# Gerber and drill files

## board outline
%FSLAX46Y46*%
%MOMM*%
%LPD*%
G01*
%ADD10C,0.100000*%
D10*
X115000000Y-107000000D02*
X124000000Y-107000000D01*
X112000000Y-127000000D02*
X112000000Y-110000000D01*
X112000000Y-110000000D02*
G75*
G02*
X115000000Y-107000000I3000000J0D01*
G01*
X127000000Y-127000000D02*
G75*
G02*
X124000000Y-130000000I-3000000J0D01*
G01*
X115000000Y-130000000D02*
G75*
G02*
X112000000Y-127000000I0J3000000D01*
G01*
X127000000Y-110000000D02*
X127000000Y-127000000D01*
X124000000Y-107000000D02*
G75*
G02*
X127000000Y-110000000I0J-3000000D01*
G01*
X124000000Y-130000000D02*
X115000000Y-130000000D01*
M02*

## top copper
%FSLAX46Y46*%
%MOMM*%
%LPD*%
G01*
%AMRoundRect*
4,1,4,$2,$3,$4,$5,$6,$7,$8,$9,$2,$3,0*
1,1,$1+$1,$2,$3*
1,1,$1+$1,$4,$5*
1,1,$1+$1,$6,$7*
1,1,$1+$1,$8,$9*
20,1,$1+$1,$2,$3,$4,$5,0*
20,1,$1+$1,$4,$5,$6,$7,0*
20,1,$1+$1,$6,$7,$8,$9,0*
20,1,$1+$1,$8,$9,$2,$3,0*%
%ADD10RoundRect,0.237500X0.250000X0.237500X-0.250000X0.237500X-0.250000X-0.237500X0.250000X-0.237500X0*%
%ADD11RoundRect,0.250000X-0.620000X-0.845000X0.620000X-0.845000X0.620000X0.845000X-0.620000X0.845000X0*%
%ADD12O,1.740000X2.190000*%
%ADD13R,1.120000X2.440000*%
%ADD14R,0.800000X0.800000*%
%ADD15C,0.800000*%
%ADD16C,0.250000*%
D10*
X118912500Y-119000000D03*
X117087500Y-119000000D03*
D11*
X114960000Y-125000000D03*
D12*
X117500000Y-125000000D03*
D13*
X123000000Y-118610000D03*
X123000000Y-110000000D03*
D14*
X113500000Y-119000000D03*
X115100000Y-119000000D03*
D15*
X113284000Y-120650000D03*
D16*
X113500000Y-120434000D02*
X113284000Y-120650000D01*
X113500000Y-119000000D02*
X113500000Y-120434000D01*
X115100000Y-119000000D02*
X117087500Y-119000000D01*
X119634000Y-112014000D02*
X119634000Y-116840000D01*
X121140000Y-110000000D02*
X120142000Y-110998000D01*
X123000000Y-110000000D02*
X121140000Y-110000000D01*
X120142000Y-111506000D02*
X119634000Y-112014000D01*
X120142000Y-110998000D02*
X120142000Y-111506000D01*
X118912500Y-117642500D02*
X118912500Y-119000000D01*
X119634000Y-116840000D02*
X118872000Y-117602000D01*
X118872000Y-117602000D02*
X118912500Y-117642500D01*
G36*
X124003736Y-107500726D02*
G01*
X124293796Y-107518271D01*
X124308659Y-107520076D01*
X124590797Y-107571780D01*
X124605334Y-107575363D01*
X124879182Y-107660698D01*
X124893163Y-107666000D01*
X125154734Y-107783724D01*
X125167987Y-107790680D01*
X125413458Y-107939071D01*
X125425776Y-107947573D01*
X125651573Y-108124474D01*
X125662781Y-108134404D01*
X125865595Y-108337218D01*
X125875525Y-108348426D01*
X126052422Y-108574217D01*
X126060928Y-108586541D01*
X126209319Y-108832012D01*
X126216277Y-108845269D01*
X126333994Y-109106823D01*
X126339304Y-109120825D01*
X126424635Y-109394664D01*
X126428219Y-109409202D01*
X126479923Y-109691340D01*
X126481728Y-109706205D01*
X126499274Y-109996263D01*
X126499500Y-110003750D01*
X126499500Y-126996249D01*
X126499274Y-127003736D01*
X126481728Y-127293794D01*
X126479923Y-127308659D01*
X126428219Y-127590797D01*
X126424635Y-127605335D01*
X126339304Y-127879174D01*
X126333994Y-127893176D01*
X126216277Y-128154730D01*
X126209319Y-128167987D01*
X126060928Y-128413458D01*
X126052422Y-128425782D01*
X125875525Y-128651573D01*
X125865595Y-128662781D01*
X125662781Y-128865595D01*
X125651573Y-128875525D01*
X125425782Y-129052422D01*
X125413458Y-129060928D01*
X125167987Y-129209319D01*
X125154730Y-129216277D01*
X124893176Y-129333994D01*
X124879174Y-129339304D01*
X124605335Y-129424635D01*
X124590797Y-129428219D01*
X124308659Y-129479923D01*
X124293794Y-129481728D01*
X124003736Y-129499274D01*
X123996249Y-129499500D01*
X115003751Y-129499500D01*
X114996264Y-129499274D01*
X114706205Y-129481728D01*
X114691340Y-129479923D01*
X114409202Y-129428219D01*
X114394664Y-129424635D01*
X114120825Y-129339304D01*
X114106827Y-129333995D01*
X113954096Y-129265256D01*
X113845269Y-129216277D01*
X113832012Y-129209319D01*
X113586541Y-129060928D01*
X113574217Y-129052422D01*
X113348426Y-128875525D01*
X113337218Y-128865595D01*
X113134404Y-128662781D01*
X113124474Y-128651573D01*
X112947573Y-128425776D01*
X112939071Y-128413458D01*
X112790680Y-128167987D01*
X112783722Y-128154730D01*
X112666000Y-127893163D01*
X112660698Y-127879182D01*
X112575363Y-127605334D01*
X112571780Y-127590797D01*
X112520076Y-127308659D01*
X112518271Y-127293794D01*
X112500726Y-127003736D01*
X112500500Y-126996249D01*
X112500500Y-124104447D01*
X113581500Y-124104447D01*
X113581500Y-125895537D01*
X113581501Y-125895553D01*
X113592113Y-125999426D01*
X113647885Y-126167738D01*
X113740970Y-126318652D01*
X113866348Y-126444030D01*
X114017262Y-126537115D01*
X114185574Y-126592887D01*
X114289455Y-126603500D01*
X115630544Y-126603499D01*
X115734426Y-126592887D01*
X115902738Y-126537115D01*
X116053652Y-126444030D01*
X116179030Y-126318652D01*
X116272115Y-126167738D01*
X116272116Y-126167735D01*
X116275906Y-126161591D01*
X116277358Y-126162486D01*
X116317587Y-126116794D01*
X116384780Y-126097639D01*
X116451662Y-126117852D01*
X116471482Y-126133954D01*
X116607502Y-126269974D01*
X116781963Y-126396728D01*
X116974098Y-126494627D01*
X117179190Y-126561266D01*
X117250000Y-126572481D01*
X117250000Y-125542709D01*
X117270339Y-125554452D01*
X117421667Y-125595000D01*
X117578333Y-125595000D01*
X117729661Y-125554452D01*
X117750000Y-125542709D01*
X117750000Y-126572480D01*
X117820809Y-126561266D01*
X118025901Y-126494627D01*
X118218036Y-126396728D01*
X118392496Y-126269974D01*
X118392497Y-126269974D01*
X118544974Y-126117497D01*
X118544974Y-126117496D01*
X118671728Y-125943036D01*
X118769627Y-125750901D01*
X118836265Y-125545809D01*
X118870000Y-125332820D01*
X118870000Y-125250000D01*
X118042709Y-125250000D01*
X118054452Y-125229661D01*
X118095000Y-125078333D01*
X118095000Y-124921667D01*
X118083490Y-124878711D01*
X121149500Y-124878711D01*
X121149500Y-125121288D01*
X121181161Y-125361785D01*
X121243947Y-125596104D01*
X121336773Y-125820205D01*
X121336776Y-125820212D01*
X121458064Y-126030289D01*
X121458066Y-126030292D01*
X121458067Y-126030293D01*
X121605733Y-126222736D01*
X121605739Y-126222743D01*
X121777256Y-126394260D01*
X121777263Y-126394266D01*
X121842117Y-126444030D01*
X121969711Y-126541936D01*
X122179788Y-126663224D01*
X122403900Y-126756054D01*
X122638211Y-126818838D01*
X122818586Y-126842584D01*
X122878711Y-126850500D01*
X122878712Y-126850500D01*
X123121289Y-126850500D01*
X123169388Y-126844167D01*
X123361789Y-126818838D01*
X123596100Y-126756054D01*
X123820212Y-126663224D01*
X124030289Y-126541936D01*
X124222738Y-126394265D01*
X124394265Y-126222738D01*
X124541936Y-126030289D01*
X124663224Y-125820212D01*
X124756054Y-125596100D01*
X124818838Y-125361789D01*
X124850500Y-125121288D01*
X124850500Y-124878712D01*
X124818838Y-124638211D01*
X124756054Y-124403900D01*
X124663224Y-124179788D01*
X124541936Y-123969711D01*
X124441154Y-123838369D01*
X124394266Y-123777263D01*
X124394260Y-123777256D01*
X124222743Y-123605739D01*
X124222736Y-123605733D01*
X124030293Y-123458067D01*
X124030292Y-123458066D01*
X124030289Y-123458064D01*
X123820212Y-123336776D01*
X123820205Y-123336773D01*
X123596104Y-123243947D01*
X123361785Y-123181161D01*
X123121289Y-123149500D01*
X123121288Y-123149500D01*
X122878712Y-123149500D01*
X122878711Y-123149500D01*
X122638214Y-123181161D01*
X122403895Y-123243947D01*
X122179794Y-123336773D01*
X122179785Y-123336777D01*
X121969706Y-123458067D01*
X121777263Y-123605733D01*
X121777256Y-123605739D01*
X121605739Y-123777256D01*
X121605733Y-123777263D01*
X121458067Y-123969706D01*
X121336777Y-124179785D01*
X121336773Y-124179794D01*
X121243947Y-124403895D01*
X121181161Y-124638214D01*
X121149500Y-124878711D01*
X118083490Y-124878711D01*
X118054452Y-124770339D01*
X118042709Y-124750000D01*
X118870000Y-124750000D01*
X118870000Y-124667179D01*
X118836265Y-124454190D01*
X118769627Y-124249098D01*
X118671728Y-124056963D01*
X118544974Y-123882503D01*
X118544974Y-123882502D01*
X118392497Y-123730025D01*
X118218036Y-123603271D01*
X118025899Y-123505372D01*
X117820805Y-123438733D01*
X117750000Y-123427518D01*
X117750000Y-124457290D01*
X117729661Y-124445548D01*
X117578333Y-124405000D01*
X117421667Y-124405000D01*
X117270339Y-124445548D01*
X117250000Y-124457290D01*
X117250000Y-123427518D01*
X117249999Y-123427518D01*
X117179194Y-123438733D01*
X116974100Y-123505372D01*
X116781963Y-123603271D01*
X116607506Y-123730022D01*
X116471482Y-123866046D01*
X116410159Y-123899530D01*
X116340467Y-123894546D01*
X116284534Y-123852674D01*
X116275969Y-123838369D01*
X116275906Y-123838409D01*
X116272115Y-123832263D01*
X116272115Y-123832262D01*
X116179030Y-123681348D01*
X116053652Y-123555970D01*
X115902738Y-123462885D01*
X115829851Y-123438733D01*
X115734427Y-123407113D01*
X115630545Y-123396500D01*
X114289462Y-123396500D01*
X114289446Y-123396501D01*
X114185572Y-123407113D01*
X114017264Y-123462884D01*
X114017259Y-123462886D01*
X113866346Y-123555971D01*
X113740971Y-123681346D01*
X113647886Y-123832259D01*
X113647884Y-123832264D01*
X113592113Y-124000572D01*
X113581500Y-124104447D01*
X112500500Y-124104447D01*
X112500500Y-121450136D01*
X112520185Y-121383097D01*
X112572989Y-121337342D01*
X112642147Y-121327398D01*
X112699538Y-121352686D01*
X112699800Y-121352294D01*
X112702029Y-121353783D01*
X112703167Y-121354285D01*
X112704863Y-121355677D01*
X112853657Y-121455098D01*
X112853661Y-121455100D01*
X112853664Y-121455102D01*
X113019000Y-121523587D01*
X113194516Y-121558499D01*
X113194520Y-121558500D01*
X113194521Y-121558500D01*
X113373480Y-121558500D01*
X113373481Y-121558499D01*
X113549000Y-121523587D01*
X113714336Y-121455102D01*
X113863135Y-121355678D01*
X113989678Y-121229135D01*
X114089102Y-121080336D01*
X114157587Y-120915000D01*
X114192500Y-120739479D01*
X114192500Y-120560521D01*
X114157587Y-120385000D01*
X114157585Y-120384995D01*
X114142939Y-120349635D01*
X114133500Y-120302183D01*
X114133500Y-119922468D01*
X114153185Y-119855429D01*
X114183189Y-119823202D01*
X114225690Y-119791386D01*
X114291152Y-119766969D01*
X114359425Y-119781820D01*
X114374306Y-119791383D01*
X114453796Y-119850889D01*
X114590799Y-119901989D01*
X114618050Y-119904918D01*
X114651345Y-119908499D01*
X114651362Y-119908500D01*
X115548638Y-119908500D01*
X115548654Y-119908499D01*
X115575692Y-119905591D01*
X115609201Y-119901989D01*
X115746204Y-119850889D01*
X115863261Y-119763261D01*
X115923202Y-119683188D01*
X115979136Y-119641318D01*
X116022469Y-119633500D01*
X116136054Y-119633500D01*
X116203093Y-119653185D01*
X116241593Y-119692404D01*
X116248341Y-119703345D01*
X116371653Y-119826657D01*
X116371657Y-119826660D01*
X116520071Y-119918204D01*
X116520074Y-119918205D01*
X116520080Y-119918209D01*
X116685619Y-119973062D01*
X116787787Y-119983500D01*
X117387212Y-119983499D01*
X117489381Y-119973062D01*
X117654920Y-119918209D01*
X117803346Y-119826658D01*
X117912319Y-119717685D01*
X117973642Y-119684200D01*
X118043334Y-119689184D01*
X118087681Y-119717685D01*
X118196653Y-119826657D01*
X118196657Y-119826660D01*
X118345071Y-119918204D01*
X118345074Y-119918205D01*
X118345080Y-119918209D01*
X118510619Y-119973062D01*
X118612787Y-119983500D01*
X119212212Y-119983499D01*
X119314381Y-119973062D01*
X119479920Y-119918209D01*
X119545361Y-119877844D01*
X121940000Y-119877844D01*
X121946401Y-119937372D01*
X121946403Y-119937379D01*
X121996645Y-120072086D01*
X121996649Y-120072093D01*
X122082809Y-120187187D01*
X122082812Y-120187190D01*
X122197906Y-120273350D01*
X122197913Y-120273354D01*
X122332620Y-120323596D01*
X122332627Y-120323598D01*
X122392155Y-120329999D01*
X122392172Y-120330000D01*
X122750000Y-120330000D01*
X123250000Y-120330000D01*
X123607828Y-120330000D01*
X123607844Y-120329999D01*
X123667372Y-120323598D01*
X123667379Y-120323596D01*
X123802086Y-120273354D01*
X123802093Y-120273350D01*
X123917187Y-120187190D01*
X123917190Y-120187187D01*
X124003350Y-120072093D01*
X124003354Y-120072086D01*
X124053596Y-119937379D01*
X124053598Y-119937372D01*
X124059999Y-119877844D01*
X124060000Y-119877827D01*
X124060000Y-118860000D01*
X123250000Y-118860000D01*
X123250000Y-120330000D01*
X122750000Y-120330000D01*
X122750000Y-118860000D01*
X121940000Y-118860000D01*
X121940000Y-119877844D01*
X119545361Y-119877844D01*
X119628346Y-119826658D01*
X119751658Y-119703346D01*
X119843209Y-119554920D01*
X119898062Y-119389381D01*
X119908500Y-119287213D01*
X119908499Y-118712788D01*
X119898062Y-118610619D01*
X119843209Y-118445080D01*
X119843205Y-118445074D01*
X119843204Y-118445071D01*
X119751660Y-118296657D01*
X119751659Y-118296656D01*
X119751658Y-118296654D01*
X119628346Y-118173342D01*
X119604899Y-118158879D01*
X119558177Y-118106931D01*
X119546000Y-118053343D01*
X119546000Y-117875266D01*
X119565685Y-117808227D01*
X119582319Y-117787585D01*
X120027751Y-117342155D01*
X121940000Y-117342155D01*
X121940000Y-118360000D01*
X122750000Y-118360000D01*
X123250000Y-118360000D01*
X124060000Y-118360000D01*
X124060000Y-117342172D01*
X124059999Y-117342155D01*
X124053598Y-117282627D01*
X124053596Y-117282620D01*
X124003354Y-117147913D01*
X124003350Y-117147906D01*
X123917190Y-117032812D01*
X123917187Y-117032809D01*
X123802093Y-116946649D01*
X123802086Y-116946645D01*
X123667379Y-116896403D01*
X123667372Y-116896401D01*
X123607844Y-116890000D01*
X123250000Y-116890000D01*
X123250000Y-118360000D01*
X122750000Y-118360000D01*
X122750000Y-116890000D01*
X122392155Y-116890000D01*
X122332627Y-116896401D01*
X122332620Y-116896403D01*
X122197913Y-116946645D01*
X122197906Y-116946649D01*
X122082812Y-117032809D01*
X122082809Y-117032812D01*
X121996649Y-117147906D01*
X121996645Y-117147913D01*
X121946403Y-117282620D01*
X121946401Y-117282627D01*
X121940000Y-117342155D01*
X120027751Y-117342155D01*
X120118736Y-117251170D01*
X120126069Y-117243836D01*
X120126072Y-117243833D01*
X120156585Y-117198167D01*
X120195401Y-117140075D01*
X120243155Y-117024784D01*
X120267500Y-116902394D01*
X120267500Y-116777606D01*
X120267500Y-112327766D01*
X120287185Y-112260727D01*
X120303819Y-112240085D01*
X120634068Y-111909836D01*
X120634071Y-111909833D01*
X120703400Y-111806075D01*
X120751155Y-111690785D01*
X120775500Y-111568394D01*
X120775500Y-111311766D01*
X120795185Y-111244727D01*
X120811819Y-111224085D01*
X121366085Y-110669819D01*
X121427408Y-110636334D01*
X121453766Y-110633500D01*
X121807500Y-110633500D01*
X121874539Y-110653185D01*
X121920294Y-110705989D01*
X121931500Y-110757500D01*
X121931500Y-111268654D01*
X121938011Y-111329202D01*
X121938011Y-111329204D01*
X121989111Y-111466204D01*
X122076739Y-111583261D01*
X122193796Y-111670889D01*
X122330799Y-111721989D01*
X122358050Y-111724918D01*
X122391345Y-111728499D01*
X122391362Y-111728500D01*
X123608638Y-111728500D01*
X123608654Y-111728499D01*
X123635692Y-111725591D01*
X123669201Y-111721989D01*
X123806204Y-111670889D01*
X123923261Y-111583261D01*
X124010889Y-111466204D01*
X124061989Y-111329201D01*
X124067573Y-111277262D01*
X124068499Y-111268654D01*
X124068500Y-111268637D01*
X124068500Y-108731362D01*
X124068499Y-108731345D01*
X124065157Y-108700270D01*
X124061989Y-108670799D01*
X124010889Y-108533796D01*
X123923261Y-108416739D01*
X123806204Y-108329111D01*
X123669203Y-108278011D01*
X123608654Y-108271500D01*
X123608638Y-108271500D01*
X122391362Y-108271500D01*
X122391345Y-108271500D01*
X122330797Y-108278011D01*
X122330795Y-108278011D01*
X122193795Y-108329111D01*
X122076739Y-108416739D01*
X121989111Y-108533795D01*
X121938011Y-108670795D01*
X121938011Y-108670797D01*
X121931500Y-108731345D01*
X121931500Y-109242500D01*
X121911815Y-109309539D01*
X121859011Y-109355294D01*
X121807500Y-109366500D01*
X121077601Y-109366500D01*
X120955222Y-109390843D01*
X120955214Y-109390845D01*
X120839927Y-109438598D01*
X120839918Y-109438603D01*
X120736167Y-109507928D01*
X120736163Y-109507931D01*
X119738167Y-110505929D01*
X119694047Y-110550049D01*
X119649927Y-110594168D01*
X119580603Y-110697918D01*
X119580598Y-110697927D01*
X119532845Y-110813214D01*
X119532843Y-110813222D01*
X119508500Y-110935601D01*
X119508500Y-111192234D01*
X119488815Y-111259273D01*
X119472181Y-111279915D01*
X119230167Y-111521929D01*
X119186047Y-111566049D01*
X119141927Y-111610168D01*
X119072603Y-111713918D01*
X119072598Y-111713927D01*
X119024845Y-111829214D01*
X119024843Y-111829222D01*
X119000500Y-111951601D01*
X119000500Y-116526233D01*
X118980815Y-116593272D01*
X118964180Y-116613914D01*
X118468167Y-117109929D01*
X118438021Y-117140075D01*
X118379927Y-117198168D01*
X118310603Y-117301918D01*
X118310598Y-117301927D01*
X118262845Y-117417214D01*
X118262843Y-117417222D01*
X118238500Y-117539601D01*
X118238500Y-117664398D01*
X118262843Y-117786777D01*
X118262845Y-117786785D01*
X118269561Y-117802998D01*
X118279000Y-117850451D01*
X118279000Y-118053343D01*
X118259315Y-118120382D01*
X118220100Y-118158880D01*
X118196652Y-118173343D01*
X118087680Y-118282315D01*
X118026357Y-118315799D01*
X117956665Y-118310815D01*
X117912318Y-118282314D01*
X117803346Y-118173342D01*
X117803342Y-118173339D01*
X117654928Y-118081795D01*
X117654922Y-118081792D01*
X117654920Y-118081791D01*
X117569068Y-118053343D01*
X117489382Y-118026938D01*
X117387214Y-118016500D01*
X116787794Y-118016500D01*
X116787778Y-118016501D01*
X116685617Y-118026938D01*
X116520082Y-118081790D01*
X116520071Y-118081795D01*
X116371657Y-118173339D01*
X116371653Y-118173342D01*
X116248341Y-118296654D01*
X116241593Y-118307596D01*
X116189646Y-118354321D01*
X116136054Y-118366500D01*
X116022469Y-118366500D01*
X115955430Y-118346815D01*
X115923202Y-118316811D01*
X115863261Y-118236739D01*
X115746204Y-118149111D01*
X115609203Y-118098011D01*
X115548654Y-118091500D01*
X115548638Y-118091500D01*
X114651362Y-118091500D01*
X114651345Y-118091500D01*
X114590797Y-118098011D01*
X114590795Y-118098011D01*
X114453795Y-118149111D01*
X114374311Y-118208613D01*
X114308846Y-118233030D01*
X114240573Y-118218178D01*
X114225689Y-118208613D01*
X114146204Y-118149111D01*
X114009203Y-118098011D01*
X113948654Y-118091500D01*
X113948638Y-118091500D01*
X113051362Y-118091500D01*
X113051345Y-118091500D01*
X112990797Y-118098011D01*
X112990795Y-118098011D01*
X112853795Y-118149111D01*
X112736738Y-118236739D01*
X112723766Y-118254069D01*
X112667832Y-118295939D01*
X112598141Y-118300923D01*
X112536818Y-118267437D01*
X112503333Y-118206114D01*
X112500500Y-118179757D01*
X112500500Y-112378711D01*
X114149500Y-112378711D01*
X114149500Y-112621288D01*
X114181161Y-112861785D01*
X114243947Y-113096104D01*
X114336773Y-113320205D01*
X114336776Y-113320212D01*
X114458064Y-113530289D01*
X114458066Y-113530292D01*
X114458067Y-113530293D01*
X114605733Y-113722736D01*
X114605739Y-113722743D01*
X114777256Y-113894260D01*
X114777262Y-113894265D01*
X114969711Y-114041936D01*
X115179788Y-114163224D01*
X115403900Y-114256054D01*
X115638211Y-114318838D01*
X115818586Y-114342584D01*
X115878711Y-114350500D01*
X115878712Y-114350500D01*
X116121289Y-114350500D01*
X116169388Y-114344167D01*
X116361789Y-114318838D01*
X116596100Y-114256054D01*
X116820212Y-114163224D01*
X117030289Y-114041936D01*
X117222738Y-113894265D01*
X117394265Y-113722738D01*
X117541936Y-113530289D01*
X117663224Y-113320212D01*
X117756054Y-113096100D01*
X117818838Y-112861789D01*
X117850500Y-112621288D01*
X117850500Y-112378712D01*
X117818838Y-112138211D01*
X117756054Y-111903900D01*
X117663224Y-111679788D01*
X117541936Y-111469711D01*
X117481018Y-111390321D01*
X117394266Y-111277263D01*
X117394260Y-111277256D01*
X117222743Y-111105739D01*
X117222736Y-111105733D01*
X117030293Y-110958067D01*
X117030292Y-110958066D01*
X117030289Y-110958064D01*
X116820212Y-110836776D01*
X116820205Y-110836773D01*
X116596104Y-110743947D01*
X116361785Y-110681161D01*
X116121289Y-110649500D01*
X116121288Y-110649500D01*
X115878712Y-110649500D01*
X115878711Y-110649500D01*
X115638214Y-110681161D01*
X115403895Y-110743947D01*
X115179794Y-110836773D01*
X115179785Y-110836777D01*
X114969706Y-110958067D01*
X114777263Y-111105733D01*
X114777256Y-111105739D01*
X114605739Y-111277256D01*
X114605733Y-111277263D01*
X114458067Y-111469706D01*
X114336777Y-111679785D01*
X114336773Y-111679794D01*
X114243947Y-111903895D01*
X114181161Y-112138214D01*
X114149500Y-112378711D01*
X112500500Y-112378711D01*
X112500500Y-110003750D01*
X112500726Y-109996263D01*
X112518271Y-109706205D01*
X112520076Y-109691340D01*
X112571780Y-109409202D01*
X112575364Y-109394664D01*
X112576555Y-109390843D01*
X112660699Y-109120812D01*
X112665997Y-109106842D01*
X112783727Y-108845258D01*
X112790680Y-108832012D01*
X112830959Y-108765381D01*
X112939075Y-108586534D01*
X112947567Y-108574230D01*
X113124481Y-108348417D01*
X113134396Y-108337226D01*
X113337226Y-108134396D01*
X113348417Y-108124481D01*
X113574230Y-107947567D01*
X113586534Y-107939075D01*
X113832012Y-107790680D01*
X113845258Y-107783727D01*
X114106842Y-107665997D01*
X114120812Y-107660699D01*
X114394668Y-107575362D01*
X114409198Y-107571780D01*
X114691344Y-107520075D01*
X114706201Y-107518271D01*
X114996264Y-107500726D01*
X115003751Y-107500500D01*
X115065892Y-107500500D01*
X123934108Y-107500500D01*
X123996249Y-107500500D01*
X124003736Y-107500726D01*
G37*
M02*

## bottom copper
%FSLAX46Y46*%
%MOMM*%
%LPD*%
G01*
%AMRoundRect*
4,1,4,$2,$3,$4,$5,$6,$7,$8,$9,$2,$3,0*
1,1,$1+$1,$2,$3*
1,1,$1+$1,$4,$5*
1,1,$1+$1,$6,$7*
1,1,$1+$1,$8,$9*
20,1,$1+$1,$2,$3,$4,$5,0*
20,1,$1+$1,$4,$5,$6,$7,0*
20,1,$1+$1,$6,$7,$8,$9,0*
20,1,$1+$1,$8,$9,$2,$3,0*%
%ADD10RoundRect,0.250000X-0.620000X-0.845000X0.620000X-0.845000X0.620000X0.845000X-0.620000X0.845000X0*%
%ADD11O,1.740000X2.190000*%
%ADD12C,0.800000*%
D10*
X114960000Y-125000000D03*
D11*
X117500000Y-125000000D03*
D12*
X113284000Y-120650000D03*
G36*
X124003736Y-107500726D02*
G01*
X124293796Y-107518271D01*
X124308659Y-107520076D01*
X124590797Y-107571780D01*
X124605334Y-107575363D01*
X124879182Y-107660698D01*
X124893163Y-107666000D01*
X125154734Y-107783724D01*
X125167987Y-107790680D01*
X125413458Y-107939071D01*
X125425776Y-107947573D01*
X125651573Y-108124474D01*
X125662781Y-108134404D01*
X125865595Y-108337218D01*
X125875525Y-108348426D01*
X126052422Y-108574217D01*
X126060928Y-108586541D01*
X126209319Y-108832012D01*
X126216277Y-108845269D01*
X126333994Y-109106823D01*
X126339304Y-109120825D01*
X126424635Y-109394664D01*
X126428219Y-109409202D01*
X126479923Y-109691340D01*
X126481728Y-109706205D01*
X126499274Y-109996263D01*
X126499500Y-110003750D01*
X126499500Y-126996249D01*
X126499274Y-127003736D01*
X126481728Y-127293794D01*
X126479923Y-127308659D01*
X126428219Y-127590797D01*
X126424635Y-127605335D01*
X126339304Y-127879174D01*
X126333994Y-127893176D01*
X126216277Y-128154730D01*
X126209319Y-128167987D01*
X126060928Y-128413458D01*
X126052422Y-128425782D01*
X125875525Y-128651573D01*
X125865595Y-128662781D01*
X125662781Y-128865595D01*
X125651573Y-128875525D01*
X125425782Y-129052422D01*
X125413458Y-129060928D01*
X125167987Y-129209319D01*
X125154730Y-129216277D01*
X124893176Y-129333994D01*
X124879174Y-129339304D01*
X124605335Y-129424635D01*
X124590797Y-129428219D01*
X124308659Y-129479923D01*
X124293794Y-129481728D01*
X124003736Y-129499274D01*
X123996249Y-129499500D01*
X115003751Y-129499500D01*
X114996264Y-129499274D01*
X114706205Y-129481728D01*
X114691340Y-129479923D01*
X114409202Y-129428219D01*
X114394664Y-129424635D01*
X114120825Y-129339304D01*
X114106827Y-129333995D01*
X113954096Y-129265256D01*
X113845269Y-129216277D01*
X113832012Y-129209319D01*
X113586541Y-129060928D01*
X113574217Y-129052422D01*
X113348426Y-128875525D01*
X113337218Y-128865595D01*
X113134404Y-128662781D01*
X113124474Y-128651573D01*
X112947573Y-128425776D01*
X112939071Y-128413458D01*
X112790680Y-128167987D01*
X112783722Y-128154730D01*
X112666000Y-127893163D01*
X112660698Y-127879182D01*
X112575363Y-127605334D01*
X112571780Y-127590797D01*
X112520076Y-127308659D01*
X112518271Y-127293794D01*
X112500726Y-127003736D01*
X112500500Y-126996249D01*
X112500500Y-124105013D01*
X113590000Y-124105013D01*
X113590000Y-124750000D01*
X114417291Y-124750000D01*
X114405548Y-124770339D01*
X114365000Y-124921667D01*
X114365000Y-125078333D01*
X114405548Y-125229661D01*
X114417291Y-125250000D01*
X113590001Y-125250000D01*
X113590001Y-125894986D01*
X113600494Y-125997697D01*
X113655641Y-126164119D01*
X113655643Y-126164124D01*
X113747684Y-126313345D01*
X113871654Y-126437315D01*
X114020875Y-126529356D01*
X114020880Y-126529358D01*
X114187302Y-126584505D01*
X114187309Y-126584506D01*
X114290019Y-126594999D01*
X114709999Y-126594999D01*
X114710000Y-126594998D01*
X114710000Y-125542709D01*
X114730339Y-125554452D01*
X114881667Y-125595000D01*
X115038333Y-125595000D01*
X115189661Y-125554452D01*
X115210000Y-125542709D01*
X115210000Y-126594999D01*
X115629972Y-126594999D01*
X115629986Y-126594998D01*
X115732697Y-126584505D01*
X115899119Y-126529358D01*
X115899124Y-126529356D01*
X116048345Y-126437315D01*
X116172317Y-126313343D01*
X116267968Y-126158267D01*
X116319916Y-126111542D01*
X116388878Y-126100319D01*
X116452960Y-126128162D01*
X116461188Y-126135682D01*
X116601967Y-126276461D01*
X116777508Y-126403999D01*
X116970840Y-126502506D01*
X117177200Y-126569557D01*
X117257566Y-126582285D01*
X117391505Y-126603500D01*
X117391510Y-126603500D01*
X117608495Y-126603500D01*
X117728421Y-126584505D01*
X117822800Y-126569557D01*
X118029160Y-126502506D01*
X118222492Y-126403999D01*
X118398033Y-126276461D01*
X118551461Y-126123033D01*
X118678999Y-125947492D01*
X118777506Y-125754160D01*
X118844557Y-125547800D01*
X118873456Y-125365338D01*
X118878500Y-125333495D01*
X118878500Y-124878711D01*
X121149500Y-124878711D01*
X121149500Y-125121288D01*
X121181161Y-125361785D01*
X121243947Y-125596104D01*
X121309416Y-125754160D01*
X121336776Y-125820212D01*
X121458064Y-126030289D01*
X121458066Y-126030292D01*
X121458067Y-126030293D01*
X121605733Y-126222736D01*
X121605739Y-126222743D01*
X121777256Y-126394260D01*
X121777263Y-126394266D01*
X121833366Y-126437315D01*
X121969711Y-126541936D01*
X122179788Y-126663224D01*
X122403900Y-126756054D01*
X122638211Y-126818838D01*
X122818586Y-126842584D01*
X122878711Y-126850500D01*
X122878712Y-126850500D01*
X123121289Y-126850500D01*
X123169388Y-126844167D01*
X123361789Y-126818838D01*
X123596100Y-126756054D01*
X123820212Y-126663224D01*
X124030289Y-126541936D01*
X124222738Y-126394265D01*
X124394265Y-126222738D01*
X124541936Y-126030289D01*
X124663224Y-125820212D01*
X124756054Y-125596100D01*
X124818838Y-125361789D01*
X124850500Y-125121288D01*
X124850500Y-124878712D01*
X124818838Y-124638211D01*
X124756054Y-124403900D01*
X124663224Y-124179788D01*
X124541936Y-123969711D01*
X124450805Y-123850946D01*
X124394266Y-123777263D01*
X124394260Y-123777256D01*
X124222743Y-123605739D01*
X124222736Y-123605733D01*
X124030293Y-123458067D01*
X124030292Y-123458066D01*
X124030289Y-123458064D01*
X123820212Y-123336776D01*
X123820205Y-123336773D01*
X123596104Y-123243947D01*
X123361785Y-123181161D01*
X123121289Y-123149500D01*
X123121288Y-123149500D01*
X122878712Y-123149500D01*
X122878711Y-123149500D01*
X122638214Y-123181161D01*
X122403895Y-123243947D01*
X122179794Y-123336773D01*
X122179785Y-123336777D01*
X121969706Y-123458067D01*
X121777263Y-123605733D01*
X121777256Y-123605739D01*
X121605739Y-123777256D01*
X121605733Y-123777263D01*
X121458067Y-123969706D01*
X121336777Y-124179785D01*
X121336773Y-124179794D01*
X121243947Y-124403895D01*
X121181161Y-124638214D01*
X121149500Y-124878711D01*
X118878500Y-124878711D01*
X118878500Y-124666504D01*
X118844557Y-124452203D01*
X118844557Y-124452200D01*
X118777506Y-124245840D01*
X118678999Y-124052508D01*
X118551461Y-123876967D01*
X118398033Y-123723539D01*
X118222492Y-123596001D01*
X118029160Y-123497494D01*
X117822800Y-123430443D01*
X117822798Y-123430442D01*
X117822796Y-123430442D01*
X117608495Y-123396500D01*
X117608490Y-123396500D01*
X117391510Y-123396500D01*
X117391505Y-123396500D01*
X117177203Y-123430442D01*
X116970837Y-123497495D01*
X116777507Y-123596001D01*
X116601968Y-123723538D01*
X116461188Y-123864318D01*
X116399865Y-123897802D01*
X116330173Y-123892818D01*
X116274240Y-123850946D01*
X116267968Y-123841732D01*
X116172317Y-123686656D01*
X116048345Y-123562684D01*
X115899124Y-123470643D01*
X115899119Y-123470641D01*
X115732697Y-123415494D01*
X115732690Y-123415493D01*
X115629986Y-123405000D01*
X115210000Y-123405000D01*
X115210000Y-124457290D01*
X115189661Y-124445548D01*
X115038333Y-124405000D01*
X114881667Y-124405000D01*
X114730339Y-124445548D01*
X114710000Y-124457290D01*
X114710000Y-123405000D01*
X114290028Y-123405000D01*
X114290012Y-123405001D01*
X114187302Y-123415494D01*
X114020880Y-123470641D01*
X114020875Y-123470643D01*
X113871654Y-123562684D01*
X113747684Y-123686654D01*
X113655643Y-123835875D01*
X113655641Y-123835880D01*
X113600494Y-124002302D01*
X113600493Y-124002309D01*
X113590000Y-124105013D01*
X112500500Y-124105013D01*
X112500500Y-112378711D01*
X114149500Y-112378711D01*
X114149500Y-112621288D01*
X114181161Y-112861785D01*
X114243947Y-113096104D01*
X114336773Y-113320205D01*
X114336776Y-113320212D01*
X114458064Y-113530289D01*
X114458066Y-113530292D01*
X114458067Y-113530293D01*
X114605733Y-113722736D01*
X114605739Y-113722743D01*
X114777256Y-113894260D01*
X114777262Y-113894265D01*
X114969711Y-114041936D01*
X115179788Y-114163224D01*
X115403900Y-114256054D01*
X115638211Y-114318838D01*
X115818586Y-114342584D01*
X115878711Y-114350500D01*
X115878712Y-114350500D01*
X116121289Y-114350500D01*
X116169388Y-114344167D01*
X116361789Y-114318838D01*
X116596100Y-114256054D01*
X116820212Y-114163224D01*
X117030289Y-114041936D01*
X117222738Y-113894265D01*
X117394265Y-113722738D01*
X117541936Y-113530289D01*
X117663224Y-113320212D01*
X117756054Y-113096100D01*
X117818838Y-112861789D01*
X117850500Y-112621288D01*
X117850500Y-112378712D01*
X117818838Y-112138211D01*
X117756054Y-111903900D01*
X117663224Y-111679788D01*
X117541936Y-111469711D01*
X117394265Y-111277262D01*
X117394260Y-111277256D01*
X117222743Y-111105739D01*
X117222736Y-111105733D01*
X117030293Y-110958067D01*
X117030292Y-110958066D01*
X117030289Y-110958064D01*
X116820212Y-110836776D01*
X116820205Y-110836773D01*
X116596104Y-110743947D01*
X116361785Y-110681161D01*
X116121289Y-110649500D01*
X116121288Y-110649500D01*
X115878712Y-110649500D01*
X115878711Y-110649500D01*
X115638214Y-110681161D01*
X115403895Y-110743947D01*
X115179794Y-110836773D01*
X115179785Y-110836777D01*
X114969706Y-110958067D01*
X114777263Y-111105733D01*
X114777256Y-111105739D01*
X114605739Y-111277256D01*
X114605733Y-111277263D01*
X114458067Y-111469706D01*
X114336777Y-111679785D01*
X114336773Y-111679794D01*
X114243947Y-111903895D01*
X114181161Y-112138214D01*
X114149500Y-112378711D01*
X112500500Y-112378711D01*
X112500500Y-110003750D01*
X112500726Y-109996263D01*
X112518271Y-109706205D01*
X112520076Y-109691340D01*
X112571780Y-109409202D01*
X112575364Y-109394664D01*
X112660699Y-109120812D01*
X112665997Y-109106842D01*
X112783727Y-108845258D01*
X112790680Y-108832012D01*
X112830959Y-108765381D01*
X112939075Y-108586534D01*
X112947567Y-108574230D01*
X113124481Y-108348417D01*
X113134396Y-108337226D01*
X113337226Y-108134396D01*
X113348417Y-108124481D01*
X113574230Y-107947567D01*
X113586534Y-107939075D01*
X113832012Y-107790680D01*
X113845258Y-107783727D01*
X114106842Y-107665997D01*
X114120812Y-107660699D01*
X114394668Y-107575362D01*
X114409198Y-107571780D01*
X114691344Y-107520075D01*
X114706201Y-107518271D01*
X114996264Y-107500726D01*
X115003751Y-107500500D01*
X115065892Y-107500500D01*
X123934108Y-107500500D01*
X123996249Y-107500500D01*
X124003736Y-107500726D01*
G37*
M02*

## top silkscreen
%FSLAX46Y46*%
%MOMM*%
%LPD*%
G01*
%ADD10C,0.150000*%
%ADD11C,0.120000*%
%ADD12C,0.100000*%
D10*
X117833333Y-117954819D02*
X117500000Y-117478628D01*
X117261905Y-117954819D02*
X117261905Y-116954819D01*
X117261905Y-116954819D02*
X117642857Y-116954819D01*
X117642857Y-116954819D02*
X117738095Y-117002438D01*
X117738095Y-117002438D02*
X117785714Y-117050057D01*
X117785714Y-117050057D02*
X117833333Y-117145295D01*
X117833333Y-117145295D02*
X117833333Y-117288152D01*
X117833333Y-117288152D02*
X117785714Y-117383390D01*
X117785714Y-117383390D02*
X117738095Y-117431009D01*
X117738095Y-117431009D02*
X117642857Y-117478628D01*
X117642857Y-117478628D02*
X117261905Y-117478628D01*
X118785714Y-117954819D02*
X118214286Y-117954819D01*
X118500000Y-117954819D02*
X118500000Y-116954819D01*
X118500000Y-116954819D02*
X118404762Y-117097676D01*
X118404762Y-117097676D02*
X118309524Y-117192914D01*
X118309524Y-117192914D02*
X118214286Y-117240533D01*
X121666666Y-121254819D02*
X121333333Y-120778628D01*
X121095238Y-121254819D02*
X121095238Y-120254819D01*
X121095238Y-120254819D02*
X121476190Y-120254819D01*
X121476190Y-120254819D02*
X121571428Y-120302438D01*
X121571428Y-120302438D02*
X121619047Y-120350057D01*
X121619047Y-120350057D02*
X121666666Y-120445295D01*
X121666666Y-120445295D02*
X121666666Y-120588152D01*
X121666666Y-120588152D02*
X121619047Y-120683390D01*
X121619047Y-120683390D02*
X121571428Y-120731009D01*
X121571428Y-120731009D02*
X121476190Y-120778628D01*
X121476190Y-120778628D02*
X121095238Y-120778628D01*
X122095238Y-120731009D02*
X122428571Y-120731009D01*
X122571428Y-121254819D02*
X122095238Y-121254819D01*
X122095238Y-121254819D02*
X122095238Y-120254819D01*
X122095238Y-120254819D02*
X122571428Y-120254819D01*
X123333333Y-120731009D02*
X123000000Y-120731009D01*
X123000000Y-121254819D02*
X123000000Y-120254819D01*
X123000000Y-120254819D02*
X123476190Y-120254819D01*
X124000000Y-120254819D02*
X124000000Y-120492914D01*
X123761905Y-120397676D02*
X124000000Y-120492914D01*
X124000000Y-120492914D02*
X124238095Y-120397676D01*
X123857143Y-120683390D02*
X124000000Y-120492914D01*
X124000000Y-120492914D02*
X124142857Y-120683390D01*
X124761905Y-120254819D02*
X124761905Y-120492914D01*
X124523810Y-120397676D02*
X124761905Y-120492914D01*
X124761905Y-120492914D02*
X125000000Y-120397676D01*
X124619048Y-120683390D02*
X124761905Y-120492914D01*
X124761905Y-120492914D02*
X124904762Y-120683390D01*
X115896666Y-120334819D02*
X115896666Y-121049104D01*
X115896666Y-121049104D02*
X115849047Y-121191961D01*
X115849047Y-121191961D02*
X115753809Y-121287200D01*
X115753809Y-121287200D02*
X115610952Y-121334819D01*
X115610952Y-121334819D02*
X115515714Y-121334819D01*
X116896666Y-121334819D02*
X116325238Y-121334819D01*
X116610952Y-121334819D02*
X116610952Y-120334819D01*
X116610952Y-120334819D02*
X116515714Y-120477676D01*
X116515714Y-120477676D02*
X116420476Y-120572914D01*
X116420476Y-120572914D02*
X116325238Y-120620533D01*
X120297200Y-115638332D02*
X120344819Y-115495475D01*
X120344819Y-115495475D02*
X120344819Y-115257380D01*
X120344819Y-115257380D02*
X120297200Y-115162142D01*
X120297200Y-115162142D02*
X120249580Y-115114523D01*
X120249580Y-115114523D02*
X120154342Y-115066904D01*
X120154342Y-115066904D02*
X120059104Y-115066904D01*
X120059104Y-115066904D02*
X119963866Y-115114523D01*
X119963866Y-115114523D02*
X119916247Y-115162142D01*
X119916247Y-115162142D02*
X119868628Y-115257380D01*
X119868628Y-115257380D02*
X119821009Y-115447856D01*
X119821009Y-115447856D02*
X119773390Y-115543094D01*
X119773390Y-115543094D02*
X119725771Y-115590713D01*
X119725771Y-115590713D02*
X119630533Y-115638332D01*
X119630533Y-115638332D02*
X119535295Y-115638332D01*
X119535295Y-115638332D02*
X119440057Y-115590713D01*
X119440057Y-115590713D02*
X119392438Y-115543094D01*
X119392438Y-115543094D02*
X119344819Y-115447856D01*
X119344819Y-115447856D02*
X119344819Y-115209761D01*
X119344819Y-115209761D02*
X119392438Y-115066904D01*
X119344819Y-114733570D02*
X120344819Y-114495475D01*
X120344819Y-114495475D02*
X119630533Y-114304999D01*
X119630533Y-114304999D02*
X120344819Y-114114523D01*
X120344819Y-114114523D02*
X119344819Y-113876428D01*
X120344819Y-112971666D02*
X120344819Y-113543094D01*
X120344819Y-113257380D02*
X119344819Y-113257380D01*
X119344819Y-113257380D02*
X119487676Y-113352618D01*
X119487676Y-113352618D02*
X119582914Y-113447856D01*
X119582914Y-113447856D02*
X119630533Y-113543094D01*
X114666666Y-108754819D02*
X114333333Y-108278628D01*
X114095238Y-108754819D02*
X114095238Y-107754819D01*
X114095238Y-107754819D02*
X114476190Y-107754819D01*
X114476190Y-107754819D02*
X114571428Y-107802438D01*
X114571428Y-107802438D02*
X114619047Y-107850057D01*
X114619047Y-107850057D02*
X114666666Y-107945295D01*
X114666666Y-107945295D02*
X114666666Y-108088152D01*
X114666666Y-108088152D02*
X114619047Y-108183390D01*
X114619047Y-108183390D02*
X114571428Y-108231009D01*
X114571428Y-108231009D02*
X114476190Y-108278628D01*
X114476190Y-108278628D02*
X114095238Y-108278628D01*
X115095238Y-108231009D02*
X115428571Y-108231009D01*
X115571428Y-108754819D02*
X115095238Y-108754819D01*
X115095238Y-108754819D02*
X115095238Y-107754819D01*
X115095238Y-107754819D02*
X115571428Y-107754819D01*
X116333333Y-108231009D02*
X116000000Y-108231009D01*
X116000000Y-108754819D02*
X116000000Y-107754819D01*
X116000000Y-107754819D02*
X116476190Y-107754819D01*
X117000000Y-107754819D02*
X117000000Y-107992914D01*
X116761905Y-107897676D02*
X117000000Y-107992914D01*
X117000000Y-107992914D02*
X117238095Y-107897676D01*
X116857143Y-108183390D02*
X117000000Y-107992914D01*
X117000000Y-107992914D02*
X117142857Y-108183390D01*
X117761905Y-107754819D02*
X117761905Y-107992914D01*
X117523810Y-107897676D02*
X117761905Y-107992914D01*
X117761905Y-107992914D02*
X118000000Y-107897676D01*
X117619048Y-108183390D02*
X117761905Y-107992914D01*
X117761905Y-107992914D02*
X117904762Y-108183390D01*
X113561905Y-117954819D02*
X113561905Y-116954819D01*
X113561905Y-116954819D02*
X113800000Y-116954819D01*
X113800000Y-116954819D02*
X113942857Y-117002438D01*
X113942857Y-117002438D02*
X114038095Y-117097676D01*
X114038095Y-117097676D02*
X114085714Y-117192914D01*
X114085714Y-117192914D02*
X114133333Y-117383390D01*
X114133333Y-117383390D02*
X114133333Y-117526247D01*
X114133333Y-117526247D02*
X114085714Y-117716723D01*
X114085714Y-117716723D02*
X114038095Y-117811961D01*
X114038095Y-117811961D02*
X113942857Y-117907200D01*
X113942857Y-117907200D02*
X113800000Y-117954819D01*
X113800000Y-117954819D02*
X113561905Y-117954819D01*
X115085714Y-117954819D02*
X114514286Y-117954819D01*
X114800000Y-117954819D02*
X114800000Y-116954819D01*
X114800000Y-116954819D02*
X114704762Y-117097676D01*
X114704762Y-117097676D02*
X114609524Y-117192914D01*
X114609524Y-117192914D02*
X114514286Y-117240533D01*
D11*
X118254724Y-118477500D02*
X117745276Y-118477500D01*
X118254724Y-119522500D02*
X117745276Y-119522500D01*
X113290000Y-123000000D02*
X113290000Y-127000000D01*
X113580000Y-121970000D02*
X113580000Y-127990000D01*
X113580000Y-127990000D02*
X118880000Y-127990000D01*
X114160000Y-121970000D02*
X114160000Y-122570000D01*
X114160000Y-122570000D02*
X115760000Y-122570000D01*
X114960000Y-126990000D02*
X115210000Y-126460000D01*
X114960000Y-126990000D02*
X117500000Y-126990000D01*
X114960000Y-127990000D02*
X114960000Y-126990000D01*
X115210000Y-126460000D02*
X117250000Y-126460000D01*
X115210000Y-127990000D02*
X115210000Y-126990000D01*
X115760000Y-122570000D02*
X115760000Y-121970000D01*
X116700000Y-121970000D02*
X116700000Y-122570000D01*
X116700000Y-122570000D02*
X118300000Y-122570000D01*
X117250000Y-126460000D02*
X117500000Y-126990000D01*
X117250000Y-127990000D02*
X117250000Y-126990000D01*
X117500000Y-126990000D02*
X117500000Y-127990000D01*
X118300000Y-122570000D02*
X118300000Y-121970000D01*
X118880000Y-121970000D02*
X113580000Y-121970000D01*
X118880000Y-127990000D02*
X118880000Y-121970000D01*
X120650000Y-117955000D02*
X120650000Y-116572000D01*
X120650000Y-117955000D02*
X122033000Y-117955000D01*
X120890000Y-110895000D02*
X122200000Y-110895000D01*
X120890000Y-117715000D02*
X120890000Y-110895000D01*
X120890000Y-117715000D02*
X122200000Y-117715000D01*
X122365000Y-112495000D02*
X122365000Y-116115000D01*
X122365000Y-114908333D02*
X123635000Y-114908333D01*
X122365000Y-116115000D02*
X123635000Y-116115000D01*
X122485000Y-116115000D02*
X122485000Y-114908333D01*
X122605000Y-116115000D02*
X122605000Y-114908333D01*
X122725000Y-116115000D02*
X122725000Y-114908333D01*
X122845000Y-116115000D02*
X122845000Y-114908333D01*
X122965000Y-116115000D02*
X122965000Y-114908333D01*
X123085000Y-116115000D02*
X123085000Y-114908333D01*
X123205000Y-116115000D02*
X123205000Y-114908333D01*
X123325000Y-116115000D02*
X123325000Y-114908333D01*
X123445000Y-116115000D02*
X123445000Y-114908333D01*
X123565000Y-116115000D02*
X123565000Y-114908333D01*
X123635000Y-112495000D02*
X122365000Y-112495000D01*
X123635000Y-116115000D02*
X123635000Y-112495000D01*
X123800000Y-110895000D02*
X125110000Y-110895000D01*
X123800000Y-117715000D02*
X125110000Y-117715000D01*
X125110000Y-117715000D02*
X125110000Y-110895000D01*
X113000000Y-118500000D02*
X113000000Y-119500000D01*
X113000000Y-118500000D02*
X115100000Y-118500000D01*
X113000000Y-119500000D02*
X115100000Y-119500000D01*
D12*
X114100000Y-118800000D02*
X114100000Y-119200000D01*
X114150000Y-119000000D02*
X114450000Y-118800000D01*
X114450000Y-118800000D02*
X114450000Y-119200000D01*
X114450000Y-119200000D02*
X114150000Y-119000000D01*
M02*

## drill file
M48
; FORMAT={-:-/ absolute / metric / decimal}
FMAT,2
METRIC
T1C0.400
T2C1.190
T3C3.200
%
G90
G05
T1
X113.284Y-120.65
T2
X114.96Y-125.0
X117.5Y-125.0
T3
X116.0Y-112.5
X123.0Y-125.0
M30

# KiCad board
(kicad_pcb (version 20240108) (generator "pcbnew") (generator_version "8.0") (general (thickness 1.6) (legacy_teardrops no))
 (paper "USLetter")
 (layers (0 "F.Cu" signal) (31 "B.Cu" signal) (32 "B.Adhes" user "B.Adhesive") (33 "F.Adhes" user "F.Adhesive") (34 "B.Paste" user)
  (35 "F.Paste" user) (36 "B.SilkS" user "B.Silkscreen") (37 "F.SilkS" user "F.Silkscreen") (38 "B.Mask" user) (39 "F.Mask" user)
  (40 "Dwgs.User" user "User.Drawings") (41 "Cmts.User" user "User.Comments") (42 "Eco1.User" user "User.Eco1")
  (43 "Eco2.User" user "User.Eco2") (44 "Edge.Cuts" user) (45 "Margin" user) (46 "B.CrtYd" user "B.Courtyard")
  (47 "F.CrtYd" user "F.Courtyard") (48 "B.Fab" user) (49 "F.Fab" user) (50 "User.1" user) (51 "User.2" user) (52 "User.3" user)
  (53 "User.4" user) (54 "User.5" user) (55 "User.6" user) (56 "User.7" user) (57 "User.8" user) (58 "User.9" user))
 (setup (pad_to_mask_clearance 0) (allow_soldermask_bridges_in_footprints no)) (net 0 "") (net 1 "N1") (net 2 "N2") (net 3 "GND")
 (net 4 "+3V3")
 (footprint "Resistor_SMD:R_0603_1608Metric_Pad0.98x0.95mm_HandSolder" (layer "F.Cu") (at 118 119 180)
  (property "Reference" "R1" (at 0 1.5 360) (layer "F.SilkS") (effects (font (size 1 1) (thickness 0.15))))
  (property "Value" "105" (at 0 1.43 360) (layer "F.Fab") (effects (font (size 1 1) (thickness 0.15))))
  (fp_line (start -0.254724 0.5225) (end 0.254724 0.5225) (stroke (width 0.12) (type solid)) (layer "F.SilkS"))
  (fp_line (start -0.254724 -0.5225) (end 0.254724 -0.5225) (stroke (width 0.12) (type solid)) (layer "F.SilkS"))
  (pad "1" smd roundrect (at -0.9125 0 180) (size 0.975 0.95) (layers "F.Cu" "F.Paste" "F.Mask") (roundrect_rratio 0.25) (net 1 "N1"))
  (pad "2" smd roundrect (at 0.9125 0 180) (size 0.975 0.95) (layers "F.Cu" "F.Paste" "F.Mask") (roundrect_rratio 0.25) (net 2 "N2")))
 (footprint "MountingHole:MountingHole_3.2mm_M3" (layer "F.Cu") (at 123 125)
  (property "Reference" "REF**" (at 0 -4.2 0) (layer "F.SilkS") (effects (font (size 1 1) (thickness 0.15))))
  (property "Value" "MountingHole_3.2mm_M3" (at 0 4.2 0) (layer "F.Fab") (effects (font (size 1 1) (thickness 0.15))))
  (pad "" np_thru_hole circle (at 0 0) (size 3.2 3.2) (drill 3.2) (layers "*.Cu" "*.Mask")))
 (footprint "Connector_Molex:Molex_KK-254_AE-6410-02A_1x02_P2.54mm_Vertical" (layer "F.Cu") (at 114.96 125)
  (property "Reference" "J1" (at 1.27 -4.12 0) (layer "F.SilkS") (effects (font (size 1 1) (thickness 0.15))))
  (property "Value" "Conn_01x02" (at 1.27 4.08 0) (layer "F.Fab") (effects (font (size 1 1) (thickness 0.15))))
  (fp_line (start -1.67 -2) (end -1.67 2) (stroke (width 0.12) (type solid)) (layer "F.SilkS"))
  (fp_line (start -1.38 -3.03) (end -1.38 2.99) (stroke (width 0.12) (type solid)) (layer "F.SilkS"))
  (fp_line (start -1.38 2.99) (end 3.92 2.99) (stroke (width 0.12) (type solid)) (layer "F.SilkS"))
  (fp_line (start -0.8 -3.03) (end -0.8 -2.43) (stroke (width 0.12) (type solid)) (layer "F.SilkS"))
  (fp_line (start -0.8 -2.43) (end 0.8 -2.43) (stroke (width 0.12) (type solid)) (layer "F.SilkS"))
  (fp_line (start 0 1.99) (end 0.25 1.46) (stroke (width 0.12) (type solid)) (layer "F.SilkS"))
  (fp_line (start 0 1.99) (end 2.54 1.99) (stroke (width 0.12) (type solid)) (layer "F.SilkS"))
  (fp_line (start 0 2.99) (end 0 1.99) (stroke (width 0.12) (type solid)) (layer "F.SilkS"))
  (fp_line (start 0.25 1.46) (end 2.29 1.46) (stroke (width 0.12) (type solid)) (layer "F.SilkS"))
  (fp_line (start 0.25 2.99) (end 0.25 1.99) (stroke (width 0.12) (type solid)) (layer "F.SilkS"))
  (fp_line (start 0.8 -2.43) (end 0.8 -3.03) (stroke (width 0.12) (type solid)) (layer "F.SilkS"))
  (fp_line (start 1.74 -3.03) (end 1.74 -2.43) (stroke (width 0.12) (type solid)) (layer "F.SilkS"))
  (fp_line (start 1.74 -2.43) (end 3.34 -2.43) (stroke (width 0.12) (type solid)) (layer "F.SilkS"))
  (fp_line (start 2.29 1.46) (end 2.54 1.99) (stroke (width 0.12) (type solid)) (layer "F.SilkS"))
  (fp_line (start 2.29 2.99) (end 2.29 1.99) (stroke (width 0.12) (type solid)) (layer "F.SilkS"))
  (fp_line (start 2.54 1.99) (end 2.54 2.99) (stroke (width 0.12) (type solid)) (layer "F.SilkS"))
  (fp_line (start 3.34 -2.43) (end 3.34 -3.03) (stroke (width 0.12) (type solid)) (layer "F.SilkS"))
  (fp_line (start 3.92 -3.03) (end -1.38 -3.03) (stroke (width 0.12) (type solid)) (layer "F.SilkS"))
  (fp_line (start 3.92 2.99) (end 3.92 -3.03) (stroke (width 0.12) (type solid)) (layer "F.SilkS"))
  (pad "1" thru_hole roundrect (at 0 0) (size 1.74 2.19) (drill 1.19) (layers "*.Cu" "*.Mask") (remove_unused_layers no)
   (roundrect_rratio 0.143678) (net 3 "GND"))
  (pad "2" thru_hole oval (at 2.54 0) (size 1.74 2.19) (drill 1.19) (layers "*.Cu" "*.Mask") (remove_unused_layers no) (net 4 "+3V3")))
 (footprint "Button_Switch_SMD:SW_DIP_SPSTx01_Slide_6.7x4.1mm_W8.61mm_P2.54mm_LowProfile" (layer "F.Cu") (at 123 114.305 90)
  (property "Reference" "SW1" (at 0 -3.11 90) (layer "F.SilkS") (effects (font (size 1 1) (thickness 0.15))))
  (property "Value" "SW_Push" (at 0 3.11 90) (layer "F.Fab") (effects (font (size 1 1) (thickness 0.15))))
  (fp_line (start -3.65 -2.35) (end -2.267 -2.35) (stroke (width 0.12) (type solid)) (layer "F.SilkS"))
  (fp_line (start -3.65 -2.35) (end -3.65 -0.967) (stroke (width 0.12) (type solid)) (layer "F.SilkS"))
  (fp_line (start 3.41 -2.11) (end 3.41 -0.8) (stroke (width 0.12) (type solid)) (layer "F.SilkS"))
  (fp_line (start -3.41 -2.11) (end 3.41 -2.11) (stroke (width 0.12) (type solid)) (layer "F.SilkS"))
  (fp_line (start -3.41 -2.11) (end -3.41 -0.8) (stroke (width 0.12) (type solid)) (layer "F.SilkS"))
  (fp_line (start 1.81 -0.635) (end -1.81 -0.635) (stroke (width 0.12) (type solid)) (layer "F.SilkS"))
  (fp_line (start -0.603333 -0.635) (end -0.603333 0.635) (stroke (width 0.12) (type solid)) (layer "F.SilkS"))
  (fp_line (start -1.81 -0.635) (end -1.81 0.635) (stroke (width 0.12) (type solid)) (layer "F.SilkS"))
  (fp_line (start -1.81 -0.515) (end -0.603333 -0.515) (stroke (width 0.12) (type solid)) (layer "F.SilkS"))
  (fp_line (start -1.81 -0.395) (end -0.603333 -0.395) (stroke (width 0.12) (type solid)) (layer "F.SilkS"))
  (fp_line (start -1.81 -0.275) (end -0.603333 -0.275) (stroke (width 0.12) (type solid)) (layer "F.SilkS"))
  (fp_line (start -1.81 -0.155) (end -0.603333 -0.155) (stroke (width 0.12) (type solid)) (layer "F.SilkS"))
  (fp_line (start -1.81 -0.035) (end -0.603333 -0.035) (stroke (width 0.12) (type solid)) (layer "F.SilkS"))
  (fp_line (start -1.81 0.085) (end -0.603333 0.085) (stroke (width 0.12) (type solid)) (layer "F.SilkS"))
  (fp_line (start -1.81 0.205) (end -0.603333 0.205) (stroke (width 0.12) (type solid)) (layer "F.SilkS"))
  (fp_line (start -1.81 0.325) (end -0.603333 0.325) (stroke (width 0.12) (type solid)) (layer "F.SilkS"))
  (fp_line (start -1.81 0.445) (end -0.603333 0.445) (stroke (width 0.12) (type solid)) (layer "F.SilkS"))
  (fp_line (start -1.81 0.565) (end -0.603333 0.565) (stroke (width 0.12) (type solid)) (layer "F.SilkS"))
  (fp_line (start 1.81 0.635) (end 1.81 -0.635) (stroke (width 0.12) (type solid)) (layer "F.SilkS"))
  (fp_line (start -1.81 0.635) (end 1.81 0.635) (stroke (width 0.12) (type solid)) (layer "F.SilkS"))
  (fp_line (start 3.41 0.8) (end 3.41 2.11) (stroke (width 0.12) (type solid)) (layer "F.SilkS"))
  (fp_line (start -3.41 0.8) (end -3.41 2.11) (stroke (width 0.12) (type solid)) (layer "F.SilkS"))
  (fp_line (start -3.41 2.11) (end 3.41 2.11) (stroke (width 0.12) (type solid)) (layer "F.SilkS"))
  (pad "1" smd rect (at -4.305 0 90) (size 2.44 1.12) (layers "F.Cu" "F.Paste" "F.Mask") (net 4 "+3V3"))
  (pad "2" smd rect (at 4.305 0 90) (size 2.44 1.12) (layers "F.Cu" "F.Paste" "F.Mask") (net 1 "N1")))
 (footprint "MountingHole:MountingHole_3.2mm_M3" (layer "F.Cu") (at 116 112.5)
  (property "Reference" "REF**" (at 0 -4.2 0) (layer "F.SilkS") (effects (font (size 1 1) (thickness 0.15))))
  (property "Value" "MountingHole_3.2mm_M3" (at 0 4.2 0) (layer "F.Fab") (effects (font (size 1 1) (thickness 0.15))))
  (pad "" np_thru_hole circle (at 0 0) (size 3.2 3.2) (drill 3.2) (layers "*.Cu" "*.Mask")))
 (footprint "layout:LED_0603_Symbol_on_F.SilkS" (layer "F.Cu") (at 114.3 119)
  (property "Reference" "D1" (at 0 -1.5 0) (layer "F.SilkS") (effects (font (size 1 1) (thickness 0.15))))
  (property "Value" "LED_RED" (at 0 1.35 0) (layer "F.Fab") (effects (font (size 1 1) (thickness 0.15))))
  (fp_line (start -1.3 -0.5) (end -1.3 0.5) (stroke (width 0.12) (type solid)) (layer "F.SilkS"))
  (fp_line (start -1.3 -0.5) (end 0.8 -0.5) (stroke (width 0.12) (type solid)) (layer "F.SilkS"))
  (fp_line (start -1.3 0.5) (end 0.8 0.5) (stroke (width 0.12) (type solid)) (layer "F.SilkS"))
  (fp_line (start -0.2 -0.2) (end -0.2 0.2) (stroke (width 0.1) (type solid)) (layer "F.SilkS"))
  (fp_line (start -0.15 0) (end 0.15 -0.2) (stroke (width 0.1) (type solid)) (layer "F.SilkS"))
  (fp_line (start 0.15 -0.2) (end 0.15 0.2) (stroke (width 0.1) (type solid)) (layer "F.SilkS"))
  (fp_line (start 0.15 0.2) (end -0.15 0) (stroke (width 0.1) (type solid)) (layer "F.SilkS"))
  (pad "1" smd rect (at -0.8 0 180) (size 0.8 0.8) (layers "F.Cu" "F.Paste" "F.Mask") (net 3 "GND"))
  (pad "2" smd rect (at 0.8 0 180) (size 0.8 0.8) (layers "F.Cu" "F.Paste" "F.Mask") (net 2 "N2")))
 (gr_line (start 115 107) (end 124 107) (stroke (width 0.1) (type default)) (layer "Edge.Cuts"))
 (gr_line (start 112 127) (end 112 110) (stroke (width 0.1) (type default)) (layer "Edge.Cuts"))
 (gr_arc (start 112 110) (mid 112.87868 107.87868) (end 115 107) (stroke (width 0.1) (type default)) (layer "Edge.Cuts"))
 (gr_arc (start 127 127) (mid 126.12132 129.12132) (end 124 130) (stroke (width 0.1) (type default)) (layer "Edge.Cuts"))
 (gr_arc (start 115 130) (mid 112.87868 129.12132) (end 112 127) (stroke (width 0.1) (type default)) (layer "Edge.Cuts"))
 (gr_line (start 127 110) (end 127 127) (stroke (width 0.1) (type default)) (layer "Edge.Cuts"))
 (gr_arc (start 124 107) (mid 126.12132 107.87868) (end 127 110) (stroke (width 0.1) (type default)) (layer "Edge.Cuts"))
 (gr_line (start 124 130) (end 115 130) (stroke (width 0.1) (type default)) (layer "Edge.Cuts"))
 (segment (start 113.5 120.434) (end 113.284 120.65) (width 0.25) (layer "F.Cu") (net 3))
 (segment (start 113.5 119) (end 113.5 120.434) (width 0.25) (layer "F.Cu") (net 3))
 (via (at 113.284 120.65) (size 0.8) (drill 0.4) (layers "F.Cu" "B.Cu") (free yes) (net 3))
 (segment (start 115.1 119) (end 117.0875 119) (width 0.25) (layer "F.Cu") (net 2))
 (segment (start 119.634 112.014) (end 119.634 116.84) (width 0.25) (layer "F.Cu") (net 1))
 (segment (start 121.14 110) (end 120.142 110.998) (width 0.25) (layer "F.Cu") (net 1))
 (segment (start 123 110) (end 121.14 110) (width 0.25) (layer "F.Cu") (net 1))
 (segment (start 120.142 111.506) (end 119.634 112.014) (width 0.25) (layer "F.Cu") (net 1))
 (segment (start 120.142 110.998) (end 120.142 111.506) (width 0.25) (layer "F.Cu") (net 1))
 (segment (start 118.9125 117.6425) (end 118.9125 119) (width 0.25) (layer "F.Cu") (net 1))
 (segment (start 119.634 116.84) (end 118.872 117.602) (width 0.25) (layer "F.Cu") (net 1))
 (segment (start 118.872 117.602) (end 118.9125 117.6425) (width 0.25) (layer "F.Cu") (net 1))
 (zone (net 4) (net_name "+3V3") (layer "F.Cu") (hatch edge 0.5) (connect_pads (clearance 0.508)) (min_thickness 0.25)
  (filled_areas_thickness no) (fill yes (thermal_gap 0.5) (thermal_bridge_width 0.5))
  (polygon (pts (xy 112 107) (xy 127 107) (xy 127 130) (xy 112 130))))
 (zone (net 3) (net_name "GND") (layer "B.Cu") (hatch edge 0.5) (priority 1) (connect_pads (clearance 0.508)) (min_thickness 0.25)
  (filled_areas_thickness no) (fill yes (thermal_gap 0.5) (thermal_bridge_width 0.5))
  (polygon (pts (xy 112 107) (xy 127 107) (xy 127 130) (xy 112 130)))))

